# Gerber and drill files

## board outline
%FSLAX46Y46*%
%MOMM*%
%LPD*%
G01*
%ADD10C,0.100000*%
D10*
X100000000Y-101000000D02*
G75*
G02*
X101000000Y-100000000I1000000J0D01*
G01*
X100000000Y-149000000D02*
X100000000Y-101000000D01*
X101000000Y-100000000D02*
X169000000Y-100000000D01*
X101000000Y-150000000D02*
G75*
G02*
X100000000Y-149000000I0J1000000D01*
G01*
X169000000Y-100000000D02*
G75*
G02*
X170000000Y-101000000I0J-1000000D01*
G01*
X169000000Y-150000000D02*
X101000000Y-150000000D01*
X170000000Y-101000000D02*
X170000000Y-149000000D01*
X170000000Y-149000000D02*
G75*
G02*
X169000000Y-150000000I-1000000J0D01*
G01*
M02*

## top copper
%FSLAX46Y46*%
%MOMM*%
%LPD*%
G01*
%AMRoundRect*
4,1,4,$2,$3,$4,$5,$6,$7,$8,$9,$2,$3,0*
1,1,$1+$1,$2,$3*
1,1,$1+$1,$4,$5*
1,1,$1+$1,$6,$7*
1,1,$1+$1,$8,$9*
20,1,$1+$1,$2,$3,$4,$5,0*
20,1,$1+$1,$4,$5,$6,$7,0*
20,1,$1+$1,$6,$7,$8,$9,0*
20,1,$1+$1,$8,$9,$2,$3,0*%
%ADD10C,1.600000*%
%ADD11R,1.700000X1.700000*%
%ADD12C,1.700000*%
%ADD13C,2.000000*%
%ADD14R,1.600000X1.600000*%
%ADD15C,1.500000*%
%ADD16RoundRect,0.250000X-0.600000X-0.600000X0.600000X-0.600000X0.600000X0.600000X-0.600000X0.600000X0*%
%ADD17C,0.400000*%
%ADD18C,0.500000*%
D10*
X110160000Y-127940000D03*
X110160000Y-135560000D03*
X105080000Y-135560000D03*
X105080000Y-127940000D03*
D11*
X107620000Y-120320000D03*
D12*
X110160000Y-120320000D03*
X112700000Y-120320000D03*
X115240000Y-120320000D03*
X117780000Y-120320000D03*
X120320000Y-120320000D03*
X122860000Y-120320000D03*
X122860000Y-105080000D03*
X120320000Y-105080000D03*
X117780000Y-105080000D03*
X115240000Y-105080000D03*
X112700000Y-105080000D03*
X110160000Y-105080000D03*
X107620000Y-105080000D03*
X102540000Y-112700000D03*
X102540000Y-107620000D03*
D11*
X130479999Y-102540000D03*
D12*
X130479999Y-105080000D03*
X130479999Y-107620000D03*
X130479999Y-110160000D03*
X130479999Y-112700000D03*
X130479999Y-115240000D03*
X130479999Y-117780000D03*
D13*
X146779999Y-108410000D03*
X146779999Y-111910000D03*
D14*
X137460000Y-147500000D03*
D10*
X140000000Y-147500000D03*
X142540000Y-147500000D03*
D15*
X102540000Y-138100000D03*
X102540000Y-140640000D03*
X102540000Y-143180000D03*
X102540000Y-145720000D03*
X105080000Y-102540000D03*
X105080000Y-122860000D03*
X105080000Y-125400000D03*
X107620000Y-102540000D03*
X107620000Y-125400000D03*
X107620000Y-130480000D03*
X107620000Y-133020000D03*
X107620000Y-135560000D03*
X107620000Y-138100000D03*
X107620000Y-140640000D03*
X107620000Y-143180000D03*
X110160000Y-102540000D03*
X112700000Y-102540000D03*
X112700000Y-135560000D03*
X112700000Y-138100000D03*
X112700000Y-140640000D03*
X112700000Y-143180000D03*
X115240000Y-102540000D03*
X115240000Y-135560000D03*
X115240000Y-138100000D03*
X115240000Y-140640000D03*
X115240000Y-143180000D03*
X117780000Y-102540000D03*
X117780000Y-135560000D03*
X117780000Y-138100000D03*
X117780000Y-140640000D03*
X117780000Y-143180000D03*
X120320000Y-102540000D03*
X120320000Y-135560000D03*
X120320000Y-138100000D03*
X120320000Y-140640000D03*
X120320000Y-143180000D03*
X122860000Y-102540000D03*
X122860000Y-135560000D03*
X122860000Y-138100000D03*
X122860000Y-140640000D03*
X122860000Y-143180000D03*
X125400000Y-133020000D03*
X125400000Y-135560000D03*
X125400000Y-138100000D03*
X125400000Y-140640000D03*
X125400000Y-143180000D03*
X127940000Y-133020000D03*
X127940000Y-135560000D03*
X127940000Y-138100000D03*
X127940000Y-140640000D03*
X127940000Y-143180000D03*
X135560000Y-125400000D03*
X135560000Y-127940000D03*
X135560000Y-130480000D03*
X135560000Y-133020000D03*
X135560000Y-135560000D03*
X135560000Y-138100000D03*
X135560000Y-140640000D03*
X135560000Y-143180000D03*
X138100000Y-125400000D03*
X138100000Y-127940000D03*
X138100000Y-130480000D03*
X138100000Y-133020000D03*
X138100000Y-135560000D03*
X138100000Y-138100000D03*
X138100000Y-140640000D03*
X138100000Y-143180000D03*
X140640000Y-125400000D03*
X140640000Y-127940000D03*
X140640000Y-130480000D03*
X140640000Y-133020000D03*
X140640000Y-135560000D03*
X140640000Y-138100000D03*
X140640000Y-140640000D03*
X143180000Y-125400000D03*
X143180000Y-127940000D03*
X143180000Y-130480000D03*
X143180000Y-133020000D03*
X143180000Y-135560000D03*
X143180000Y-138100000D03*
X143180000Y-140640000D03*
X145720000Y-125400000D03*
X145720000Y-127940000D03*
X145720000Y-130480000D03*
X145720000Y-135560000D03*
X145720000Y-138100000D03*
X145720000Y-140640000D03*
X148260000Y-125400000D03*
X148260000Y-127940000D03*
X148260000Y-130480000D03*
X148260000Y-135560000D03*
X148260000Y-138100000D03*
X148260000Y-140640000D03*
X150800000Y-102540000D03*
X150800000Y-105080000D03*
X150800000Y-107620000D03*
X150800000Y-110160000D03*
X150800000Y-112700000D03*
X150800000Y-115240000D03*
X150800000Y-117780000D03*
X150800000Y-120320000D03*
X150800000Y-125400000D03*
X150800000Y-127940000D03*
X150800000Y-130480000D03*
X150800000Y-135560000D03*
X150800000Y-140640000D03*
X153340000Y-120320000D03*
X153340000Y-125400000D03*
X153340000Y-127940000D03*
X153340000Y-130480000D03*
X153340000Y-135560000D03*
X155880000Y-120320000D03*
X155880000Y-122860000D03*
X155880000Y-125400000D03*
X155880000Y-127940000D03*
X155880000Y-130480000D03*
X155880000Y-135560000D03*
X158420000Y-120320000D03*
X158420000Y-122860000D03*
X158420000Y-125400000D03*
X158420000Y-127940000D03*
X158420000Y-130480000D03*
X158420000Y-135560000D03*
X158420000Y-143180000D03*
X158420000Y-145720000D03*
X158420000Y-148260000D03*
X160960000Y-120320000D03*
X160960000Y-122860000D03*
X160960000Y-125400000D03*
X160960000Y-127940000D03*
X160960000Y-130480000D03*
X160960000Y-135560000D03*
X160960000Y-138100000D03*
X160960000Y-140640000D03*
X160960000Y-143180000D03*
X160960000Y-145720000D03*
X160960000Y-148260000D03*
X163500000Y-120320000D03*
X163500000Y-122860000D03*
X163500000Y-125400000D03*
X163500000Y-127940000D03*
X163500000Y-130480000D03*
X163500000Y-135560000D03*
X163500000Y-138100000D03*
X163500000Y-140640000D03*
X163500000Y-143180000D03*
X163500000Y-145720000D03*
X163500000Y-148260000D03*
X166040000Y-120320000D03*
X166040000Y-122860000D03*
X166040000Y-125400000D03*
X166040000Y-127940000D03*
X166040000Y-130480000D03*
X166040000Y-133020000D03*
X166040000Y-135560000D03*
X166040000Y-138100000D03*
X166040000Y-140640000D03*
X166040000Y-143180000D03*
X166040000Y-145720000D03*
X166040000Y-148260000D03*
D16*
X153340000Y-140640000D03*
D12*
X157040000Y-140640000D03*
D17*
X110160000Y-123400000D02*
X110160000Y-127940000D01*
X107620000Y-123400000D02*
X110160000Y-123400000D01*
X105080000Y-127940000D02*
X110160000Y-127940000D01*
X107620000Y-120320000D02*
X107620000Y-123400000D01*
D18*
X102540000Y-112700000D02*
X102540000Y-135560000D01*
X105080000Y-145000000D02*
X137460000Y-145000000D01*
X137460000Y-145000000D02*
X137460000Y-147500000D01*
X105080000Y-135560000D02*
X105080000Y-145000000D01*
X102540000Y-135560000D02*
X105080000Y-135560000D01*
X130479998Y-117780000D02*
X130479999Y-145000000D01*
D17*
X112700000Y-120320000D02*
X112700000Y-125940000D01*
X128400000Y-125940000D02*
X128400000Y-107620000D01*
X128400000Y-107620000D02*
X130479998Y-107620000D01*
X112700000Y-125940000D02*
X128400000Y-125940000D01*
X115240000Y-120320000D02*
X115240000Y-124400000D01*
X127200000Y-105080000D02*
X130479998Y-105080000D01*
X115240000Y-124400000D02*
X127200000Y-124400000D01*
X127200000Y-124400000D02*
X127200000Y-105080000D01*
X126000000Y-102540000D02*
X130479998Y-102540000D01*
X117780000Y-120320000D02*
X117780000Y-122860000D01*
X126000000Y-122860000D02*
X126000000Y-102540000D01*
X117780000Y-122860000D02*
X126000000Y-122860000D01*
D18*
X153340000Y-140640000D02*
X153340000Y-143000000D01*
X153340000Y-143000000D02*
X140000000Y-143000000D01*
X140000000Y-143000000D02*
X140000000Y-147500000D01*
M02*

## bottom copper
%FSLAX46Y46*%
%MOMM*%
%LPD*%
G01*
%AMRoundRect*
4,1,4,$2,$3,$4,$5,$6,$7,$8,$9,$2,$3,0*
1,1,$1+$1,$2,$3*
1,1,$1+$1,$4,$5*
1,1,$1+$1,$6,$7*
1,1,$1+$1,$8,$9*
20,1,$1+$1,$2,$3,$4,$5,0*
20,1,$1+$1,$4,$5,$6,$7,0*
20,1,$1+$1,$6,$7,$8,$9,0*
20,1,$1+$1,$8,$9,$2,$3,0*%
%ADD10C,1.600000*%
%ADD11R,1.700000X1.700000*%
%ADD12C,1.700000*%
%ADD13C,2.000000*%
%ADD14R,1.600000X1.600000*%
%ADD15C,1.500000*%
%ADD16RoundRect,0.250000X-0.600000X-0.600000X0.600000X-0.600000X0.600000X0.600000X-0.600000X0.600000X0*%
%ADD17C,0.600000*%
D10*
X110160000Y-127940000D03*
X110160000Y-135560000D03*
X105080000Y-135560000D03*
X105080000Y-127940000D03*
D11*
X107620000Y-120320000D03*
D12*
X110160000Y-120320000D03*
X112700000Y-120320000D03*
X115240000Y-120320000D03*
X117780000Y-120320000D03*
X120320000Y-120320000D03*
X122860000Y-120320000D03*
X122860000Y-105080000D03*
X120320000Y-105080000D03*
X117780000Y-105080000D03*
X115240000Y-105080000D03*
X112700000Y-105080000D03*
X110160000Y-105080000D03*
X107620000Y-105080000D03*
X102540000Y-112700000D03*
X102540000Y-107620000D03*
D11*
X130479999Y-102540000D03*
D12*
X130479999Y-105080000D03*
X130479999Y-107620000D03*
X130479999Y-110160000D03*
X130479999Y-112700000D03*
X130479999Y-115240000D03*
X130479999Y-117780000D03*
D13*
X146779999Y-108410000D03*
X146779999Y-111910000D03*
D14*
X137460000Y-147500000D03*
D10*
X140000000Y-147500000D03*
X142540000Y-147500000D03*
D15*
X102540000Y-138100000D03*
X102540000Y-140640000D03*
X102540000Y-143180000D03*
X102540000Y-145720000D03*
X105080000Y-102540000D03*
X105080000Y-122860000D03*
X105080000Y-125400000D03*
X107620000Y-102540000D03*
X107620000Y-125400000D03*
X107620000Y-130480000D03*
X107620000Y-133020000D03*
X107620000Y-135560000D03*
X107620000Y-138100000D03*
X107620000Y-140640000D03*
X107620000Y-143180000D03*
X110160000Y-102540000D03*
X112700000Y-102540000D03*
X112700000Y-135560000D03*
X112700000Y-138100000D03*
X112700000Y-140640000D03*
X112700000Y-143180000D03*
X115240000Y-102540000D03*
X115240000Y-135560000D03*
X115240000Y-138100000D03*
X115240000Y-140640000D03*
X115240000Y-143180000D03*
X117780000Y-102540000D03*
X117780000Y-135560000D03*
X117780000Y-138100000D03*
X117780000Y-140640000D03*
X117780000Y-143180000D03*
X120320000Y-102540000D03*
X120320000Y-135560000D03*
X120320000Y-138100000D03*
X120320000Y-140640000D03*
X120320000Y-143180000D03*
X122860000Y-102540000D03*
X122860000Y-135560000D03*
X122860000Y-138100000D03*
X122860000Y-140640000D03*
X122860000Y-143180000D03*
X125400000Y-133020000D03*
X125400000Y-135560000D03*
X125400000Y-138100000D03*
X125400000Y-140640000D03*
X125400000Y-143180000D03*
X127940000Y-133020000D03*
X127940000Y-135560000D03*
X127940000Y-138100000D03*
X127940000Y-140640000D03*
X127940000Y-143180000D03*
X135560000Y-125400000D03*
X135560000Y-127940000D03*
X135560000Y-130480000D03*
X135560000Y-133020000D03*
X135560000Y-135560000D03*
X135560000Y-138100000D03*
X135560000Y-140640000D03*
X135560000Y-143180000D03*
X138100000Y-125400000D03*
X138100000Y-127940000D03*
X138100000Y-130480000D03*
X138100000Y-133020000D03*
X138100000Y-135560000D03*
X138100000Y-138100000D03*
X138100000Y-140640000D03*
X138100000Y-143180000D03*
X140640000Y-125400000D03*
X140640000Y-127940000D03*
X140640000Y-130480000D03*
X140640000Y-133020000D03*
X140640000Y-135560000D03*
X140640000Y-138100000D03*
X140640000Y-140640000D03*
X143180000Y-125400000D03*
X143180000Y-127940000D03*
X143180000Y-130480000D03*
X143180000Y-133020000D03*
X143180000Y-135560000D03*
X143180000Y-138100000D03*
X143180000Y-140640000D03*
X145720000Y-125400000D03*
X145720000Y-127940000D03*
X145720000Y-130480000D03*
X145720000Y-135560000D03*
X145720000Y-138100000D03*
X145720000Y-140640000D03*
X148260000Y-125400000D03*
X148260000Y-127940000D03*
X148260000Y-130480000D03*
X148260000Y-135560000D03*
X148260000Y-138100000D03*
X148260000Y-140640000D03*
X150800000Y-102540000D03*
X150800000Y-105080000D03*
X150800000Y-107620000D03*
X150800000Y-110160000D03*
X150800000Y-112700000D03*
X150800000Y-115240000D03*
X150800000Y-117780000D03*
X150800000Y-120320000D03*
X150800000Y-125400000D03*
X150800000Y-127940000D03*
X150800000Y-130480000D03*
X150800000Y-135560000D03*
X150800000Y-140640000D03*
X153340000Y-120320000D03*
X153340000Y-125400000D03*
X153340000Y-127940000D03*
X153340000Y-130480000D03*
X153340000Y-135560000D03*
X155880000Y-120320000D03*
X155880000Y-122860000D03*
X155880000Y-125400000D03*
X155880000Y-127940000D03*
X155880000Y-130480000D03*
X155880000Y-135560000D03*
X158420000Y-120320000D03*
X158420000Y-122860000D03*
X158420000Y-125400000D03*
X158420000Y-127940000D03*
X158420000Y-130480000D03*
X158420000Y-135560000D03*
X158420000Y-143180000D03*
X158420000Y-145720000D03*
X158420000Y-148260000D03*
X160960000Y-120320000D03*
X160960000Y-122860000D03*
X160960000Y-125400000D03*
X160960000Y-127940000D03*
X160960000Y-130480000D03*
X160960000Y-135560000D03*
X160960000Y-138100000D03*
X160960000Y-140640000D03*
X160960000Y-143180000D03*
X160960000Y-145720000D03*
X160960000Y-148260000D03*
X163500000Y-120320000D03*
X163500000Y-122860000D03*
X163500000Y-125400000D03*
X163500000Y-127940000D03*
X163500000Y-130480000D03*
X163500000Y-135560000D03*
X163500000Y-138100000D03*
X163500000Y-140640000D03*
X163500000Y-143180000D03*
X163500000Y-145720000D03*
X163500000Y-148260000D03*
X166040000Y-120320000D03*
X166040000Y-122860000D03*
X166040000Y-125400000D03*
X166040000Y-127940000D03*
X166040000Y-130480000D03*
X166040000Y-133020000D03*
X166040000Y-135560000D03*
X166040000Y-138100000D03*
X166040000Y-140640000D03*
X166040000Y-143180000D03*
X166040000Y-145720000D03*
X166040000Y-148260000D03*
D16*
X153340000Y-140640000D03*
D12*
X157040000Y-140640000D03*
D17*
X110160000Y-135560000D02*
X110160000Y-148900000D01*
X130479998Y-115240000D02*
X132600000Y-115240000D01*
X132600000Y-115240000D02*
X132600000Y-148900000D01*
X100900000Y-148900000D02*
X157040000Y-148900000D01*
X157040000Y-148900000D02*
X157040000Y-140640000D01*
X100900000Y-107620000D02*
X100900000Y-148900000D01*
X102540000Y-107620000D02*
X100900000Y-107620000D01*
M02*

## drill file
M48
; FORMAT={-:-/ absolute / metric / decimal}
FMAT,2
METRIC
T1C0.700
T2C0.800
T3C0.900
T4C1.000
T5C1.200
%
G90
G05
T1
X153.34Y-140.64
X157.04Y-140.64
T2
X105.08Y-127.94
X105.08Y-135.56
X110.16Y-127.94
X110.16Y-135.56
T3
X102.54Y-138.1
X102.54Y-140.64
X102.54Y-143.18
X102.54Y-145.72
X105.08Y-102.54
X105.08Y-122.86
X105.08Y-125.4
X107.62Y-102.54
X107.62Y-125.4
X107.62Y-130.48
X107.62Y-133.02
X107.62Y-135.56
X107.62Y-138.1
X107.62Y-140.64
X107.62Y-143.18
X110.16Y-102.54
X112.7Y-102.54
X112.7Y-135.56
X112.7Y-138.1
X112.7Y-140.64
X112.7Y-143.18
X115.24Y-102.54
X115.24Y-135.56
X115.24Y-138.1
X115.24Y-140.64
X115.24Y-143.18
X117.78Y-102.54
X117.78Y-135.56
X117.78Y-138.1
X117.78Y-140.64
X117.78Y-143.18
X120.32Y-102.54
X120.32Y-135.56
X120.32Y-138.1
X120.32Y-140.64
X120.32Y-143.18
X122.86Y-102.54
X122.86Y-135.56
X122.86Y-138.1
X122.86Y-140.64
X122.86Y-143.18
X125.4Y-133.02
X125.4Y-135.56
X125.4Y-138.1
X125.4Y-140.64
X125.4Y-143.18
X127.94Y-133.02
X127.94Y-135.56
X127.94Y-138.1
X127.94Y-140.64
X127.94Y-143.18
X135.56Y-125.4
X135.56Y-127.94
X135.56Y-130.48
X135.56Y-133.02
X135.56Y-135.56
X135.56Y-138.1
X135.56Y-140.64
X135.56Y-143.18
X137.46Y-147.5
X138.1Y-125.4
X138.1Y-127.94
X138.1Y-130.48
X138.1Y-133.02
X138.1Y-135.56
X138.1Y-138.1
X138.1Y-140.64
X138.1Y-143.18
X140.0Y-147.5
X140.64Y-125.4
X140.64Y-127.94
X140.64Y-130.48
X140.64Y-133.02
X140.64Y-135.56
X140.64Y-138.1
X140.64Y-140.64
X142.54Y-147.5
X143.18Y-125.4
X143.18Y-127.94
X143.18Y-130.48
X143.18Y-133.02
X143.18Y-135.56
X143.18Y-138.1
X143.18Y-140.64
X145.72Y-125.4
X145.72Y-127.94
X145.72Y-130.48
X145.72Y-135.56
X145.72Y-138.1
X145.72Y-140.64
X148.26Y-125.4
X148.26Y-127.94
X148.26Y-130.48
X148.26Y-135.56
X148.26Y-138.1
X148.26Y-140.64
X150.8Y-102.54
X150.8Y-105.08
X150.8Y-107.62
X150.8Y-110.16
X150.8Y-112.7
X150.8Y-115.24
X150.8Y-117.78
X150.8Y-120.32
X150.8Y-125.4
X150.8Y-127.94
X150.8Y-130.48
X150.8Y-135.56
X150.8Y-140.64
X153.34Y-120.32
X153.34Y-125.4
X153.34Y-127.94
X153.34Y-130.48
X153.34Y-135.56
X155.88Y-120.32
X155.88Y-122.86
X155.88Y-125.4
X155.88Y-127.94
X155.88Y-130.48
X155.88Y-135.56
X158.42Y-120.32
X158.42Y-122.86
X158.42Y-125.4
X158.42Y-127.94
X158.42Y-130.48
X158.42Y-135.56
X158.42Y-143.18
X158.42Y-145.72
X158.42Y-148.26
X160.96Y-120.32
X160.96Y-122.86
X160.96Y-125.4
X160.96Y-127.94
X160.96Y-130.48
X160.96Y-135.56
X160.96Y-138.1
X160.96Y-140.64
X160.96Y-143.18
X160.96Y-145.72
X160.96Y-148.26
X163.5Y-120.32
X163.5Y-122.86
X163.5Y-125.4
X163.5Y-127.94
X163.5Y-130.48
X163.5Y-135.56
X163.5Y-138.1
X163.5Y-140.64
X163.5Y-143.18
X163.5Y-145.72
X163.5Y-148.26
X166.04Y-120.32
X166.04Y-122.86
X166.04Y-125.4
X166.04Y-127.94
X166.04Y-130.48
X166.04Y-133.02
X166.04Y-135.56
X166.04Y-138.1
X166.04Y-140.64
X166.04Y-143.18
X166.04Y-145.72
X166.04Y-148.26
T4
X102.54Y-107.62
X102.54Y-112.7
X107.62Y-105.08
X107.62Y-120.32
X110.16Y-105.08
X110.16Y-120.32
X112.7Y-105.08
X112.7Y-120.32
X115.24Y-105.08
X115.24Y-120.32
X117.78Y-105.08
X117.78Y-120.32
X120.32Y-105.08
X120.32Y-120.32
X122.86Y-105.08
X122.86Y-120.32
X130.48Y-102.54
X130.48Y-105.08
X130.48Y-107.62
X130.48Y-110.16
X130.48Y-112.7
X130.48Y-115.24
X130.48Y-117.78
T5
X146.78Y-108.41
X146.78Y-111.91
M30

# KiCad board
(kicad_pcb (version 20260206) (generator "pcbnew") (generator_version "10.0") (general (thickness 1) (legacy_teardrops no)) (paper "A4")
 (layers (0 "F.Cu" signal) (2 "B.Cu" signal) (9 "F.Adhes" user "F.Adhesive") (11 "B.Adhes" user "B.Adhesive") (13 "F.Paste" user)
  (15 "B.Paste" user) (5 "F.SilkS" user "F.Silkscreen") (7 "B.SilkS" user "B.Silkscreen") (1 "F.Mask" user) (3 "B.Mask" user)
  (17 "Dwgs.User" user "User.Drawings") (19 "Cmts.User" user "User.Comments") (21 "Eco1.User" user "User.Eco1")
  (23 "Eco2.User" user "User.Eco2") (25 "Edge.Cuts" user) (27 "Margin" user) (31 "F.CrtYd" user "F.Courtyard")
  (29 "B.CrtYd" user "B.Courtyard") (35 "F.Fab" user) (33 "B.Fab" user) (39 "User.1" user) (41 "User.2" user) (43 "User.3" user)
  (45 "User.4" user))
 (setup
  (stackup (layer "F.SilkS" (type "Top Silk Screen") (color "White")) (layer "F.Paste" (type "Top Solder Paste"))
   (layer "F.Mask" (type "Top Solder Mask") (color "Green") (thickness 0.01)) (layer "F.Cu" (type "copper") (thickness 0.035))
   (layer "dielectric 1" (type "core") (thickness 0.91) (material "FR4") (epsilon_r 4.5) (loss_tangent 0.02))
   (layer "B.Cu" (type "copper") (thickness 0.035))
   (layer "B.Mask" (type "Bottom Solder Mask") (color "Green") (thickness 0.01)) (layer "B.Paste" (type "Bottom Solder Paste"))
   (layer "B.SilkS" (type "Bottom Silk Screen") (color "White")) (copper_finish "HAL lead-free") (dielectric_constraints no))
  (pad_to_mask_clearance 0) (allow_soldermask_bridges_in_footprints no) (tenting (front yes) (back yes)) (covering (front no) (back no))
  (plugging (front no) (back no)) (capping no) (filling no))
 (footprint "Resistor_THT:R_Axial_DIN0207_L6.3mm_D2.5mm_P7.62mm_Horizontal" (layer "F.Cu") (at 110.16 127.94 -90)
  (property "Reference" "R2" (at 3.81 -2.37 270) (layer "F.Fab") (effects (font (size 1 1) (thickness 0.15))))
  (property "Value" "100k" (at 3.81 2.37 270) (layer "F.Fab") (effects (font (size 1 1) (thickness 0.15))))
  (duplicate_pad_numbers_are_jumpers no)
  (pad "1" thru_hole circle (at 0 0 270) (size 1.6 1.6) (drill 0.8) (layers "*.Cu" "*.Mask") (remove_unused_layers no) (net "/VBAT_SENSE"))
  (pad "2" thru_hole circle (at 7.62 0 270) (size 1.6 1.6) (drill 0.8) (layers "*.Cu" "*.Mask") (remove_unused_layers no) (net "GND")))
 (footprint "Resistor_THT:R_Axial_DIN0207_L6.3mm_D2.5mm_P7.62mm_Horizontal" (layer "F.Cu") (at 105.08 135.56 90)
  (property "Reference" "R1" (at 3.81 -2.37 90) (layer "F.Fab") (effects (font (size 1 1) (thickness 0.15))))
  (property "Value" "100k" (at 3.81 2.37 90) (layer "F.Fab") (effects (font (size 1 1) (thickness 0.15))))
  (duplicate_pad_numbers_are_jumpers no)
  (pad "1" thru_hole circle (at 0 0 90) (size 1.6 1.6) (drill 0.8) (layers "*.Cu" "*.Mask") (remove_unused_layers no) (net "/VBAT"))
  (pad "2" thru_hole circle (at 7.62 0 90) (size 1.6 1.6) (drill 0.8) (layers "*.Cu" "*.Mask") (remove_unused_layers no) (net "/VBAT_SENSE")))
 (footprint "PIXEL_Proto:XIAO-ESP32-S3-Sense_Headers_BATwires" (layer "F.Cu") (at 115.24 112.7 180)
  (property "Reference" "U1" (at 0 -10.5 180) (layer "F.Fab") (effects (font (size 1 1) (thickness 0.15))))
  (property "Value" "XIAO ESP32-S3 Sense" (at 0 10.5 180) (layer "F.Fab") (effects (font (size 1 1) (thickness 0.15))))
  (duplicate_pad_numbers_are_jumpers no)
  (pad "1" thru_hole rect (at 7.62 -7.62 180) (size 1.7 1.7) (drill 1) (layers "*.Cu" "*.Mask") (remove_unused_layers no)
   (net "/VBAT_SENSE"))
  (pad "2" thru_hole circle (at 5.08 -7.62 180) (size 1.7 1.7) (drill 1) (layers "*.Cu" "*.Mask") (remove_unused_layers no)
   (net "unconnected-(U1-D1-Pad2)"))
  (pad "3" thru_hole circle (at 2.54 -7.62 180) (size 1.7 1.7) (drill 1) (layers "*.Cu" "*.Mask") (remove_unused_layers no)
   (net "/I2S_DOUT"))
  (pad "4" thru_hole circle (at 0 -7.62 180) (size 1.7 1.7) (drill 1) (layers "*.Cu" "*.Mask") (remove_unused_layers no) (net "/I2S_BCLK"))
  (pad "5" thru_hole circle (at -2.54 -7.62 180) (size 1.7 1.7) (drill 1) (layers "*.Cu" "*.Mask") (remove_unused_layers no)
   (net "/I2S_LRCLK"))
  (pad "6" thru_hole circle (at -5.08 -7.62 180) (size 1.7 1.7) (drill 1) (layers "*.Cu" "*.Mask") (remove_unused_layers no)
   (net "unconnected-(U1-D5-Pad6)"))
  (pad "7" thru_hole circle (at -7.62 -7.62 180) (size 1.7 1.7) (drill 1) (layers "*.Cu" "*.Mask") (remove_unused_layers no)
   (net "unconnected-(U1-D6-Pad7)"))
  (pad "8" thru_hole circle (at -7.62 7.62 180) (size 1.7 1.7) (drill 1) (layers "*.Cu" "*.Mask") (remove_unused_layers no)
   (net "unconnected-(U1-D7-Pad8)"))
  (pad "9" thru_hole circle (at -5.08 7.62 180) (size 1.7 1.7) (drill 1) (layers "*.Cu" "*.Mask") (remove_unused_layers no)
   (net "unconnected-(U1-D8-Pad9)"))
  (pad "10" thru_hole circle (at -2.54 7.62 180) (size 1.7 1.7) (drill 1) (layers "*.Cu" "*.Mask") (remove_unused_layers no)
   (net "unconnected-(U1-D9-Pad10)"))
  (pad "11" thru_hole circle (at 0 7.62 180) (size 1.7 1.7) (drill 1) (layers "*.Cu" "*.Mask") (remove_unused_layers no)
   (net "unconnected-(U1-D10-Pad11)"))
  (pad "12" thru_hole circle (at 2.54 7.62 180) (size 1.7 1.7) (drill 1) (layers "*.Cu" "*.Mask") (remove_unused_layers no)
   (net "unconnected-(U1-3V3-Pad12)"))
  (pad "13" thru_hole circle (at 5.08 7.62 180) (size 1.7 1.7) (drill 1) (layers "*.Cu" "*.Mask") (remove_unused_layers no)
   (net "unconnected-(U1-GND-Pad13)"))
  (pad "14" thru_hole circle (at 7.62 7.62 180) (size 1.7 1.7) (drill 1) (layers "*.Cu" "*.Mask") (remove_unused_layers no)
   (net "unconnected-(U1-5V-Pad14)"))
  (pad "23" thru_hole circle (at 12.7 0 180) (size 1.7 1.7) (drill 1) (layers "*.Cu" "*.Mask") (remove_unused_layers no) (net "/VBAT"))
  (pad "24" thru_hole circle (at 12.7 5.08 180) (size 1.7 1.7) (drill 1) (layers "*.Cu" "*.Mask") (remove_unused_layers no) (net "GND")))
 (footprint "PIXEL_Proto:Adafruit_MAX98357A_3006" (layer "F.Cu") (at 130.479999 102.54)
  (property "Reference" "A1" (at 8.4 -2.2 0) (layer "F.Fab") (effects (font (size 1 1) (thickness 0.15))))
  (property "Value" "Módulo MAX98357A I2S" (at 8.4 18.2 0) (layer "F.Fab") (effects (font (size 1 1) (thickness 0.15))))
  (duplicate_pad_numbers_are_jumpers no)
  (pad "1" thru_hole rect (at 0 0) (size 1.7 1.7) (drill 1) (layers "*.Cu" "*.Mask") (remove_unused_layers no) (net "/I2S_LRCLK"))
  (pad "2" thru_hole circle (at 0 2.54) (size 1.7 1.7) (drill 1) (layers "*.Cu" "*.Mask") (remove_unused_layers no) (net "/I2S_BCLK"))
  (pad "3" thru_hole circle (at 0 5.08) (size 1.7 1.7) (drill 1) (layers "*.Cu" "*.Mask") (remove_unused_layers no) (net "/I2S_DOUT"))
  (pad "4" thru_hole circle (at 0 7.62) (size 1.7 1.7) (drill 1) (layers "*.Cu" "*.Mask") (remove_unused_layers no)
   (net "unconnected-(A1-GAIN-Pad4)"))
  (pad "5" thru_hole circle (at 0 10.16) (size 1.7 1.7) (drill 1) (layers "*.Cu" "*.Mask") (remove_unused_layers no)
   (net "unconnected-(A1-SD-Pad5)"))
  (pad "6" thru_hole circle (at 0 12.7) (size 1.7 1.7) (drill 1) (layers "*.Cu" "*.Mask") (remove_unused_layers no) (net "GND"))
  (pad "7" thru_hole circle (at 0 15.24) (size 1.7 1.7) (drill 1) (layers "*.Cu" "*.Mask") (remove_unused_layers no) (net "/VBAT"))
  (pad "8" thru_hole circle (at 16.3 5.87) (size 2 2) (drill 1.2) (layers "*.Cu" "*.Mask") (remove_unused_layers no) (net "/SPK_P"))
  (pad "9" thru_hole circle (at 16.3 9.37) (size 2 2) (drill 1.2) (layers "*.Cu" "*.Mask") (remove_unused_layers no) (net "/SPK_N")))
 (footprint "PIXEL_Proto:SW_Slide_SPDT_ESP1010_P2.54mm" (layer "F.Cu") (at 140 147.5)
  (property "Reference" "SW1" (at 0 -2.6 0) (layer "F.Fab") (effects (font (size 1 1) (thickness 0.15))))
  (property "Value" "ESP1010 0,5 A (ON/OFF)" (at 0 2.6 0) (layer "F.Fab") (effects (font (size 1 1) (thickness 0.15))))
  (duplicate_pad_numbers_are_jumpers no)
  (pad "1" thru_hole rect (at -2.54 0) (size 1.6 1.6) (drill 0.9) (layers "*.Cu" "*.Mask") (remove_unused_layers no) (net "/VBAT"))
  (pad "2" thru_hole circle (at 0 0) (size 1.6 1.6) (drill 0.9) (layers "*.Cu" "*.Mask") (remove_unused_layers no) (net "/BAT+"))
  (pad "3" thru_hole circle (at 2.54 0) (size 1.6 1.6) (drill 0.9) (layers "*.Cu" "*.Mask") (remove_unused_layers no)
   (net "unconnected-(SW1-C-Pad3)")))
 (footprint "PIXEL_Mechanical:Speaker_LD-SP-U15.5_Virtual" (layer "F.Cu") (at 161 108.2)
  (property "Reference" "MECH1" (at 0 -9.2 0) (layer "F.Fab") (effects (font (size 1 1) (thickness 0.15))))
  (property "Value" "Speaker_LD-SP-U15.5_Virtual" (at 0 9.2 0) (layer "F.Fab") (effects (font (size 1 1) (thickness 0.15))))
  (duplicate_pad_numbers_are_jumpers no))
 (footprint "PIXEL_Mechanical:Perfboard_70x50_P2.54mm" (layer "F.Cu") (at 0 0)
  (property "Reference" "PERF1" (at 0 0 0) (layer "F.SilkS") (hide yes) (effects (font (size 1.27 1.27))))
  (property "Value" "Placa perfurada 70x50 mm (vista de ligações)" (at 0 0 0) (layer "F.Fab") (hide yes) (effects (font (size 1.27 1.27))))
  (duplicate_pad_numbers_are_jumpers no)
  (pad "" thru_hole circle (at 102.54 138.1) (size 1.5 1.5) (drill 0.9) (layers "*.Cu" "*.Mask") (remove_unused_layers no))
  (pad "" thru_hole circle (at 102.54 140.64) (size 1.5 1.5) (drill 0.9) (layers "*.Cu" "*.Mask") (remove_unused_layers no))
  (pad "" thru_hole circle (at 102.54 143.18) (size 1.5 1.5) (drill 0.9) (layers "*.Cu" "*.Mask") (remove_unused_layers no))
  (pad "" thru_hole circle (at 102.54 145.72) (size 1.5 1.5) (drill 0.9) (layers "*.Cu" "*.Mask") (remove_unused_layers no))
  (pad "" thru_hole circle (at 105.08 102.54) (size 1.5 1.5) (drill 0.9) (layers "*.Cu" "*.Mask") (remove_unused_layers no))
  (pad "" thru_hole circle (at 105.08 122.86) (size 1.5 1.5) (drill 0.9) (layers "*.Cu" "*.Mask") (remove_unused_layers no))
  (pad "" thru_hole circle (at 105.08 125.4) (size 1.5 1.5) (drill 0.9) (layers "*.Cu" "*.Mask") (remove_unused_layers no))
  (pad "" thru_hole circle (at 107.62 102.54) (size 1.5 1.5) (drill 0.9) (layers "*.Cu" "*.Mask") (remove_unused_layers no))
  (pad "" thru_hole circle (at 107.62 125.4) (size 1.5 1.5) (drill 0.9) (layers "*.Cu" "*.Mask") (remove_unused_layers no))
  (pad "" thru_hole circle (at 107.62 130.48) (size 1.5 1.5) (drill 0.9) (layers "*.Cu" "*.Mask") (remove_unused_layers no))
  (pad "" thru_hole circle (at 107.62 133.02) (size 1.5 1.5) (drill 0.9) (layers "*.Cu" "*.Mask") (remove_unused_layers no))
  (pad "" thru_hole circle (at 107.62 135.56) (size 1.5 1.5) (drill 0.9) (layers "*.Cu" "*.Mask") (remove_unused_layers no))
  (pad "" thru_hole circle (at 107.62 138.1) (size 1.5 1.5) (drill 0.9) (layers "*.Cu" "*.Mask") (remove_unused_layers no))
  (pad "" thru_hole circle (at 107.62 140.64) (size 1.5 1.5) (drill 0.9) (layers "*.Cu" "*.Mask") (remove_unused_layers no))
  (pad "" thru_hole circle (at 107.62 143.18) (size 1.5 1.5) (drill 0.9) (layers "*.Cu" "*.Mask") (remove_unused_layers no))
  (pad "" thru_hole circle (at 110.16 102.54) (size 1.5 1.5) (drill 0.9) (layers "*.Cu" "*.Mask") (remove_unused_layers no))
  (pad "" thru_hole circle (at 112.7 102.54) (size 1.5 1.5) (drill 0.9) (layers "*.Cu" "*.Mask") (remove_unused_layers no))
  (pad "" thru_hole circle (at 112.7 135.56) (size 1.5 1.5) (drill 0.9) (layers "*.Cu" "*.Mask") (remove_unused_layers no))
  (pad "" thru_hole circle (at 112.7 138.1) (size 1.5 1.5) (drill 0.9) (layers "*.Cu" "*.Mask") (remove_unused_layers no))
  (pad "" thru_hole circle (at 112.7 140.64) (size 1.5 1.5) (drill 0.9) (layers "*.Cu" "*.Mask") (remove_unused_layers no))
  (pad "" thru_hole circle (at 112.7 143.18) (size 1.5 1.5) (drill 0.9) (layers "*.Cu" "*.Mask") (remove_unused_layers no))
  (pad "" thru_hole circle (at 115.24 102.54) (size 1.5 1.5) (drill 0.9) (layers "*.Cu" "*.Mask") (remove_unused_layers no))
  (pad "" thru_hole circle (at 115.24 135.56) (size 1.5 1.5) (drill 0.9) (layers "*.Cu" "*.Mask") (remove_unused_layers no))
  (pad "" thru_hole circle (at 115.24 138.1) (size 1.5 1.5) (drill 0.9) (layers "*.Cu" "*.Mask") (remove_unused_layers no))
  (pad "" thru_hole circle (at 115.24 140.64) (size 1.5 1.5) (drill 0.9) (layers "*.Cu" "*.Mask") (remove_unused_layers no))
  (pad "" thru_hole circle (at 115.24 143.18) (size 1.5 1.5) (drill 0.9) (layers "*.Cu" "*.Mask") (remove_unused_layers no))
  (pad "" thru_hole circle (at 117.78 102.54) (size 1.5 1.5) (drill 0.9) (layers "*.Cu" "*.Mask") (remove_unused_layers no))
  (pad "" thru_hole circle (at 117.78 135.56) (size 1.5 1.5) (drill 0.9) (layers "*.Cu" "*.Mask") (remove_unused_layers no))
  (pad "" thru_hole circle (at 117.78 138.1) (size 1.5 1.5) (drill 0.9) (layers "*.Cu" "*.Mask") (remove_unused_layers no))
  (pad "" thru_hole circle (at 117.78 140.64) (size 1.5 1.5) (drill 0.9) (layers "*.Cu" "*.Mask") (remove_unused_layers no))
  (pad "" thru_hole circle (at 117.78 143.18) (size 1.5 1.5) (drill 0.9) (layers "*.Cu" "*.Mask") (remove_unused_layers no))
  (pad "" thru_hole circle (at 120.32 102.54) (size 1.5 1.5) (drill 0.9) (layers "*.Cu" "*.Mask") (remove_unused_layers no))
  (pad "" thru_hole circle (at 120.32 135.56) (size 1.5 1.5) (drill 0.9) (layers "*.Cu" "*.Mask") (remove_unused_layers no))
  (pad "" thru_hole circle (at 120.32 138.1) (size 1.5 1.5) (drill 0.9) (layers "*.Cu" "*.Mask") (remove_unused_layers no))
  (pad "" thru_hole circle (at 120.32 140.64) (size 1.5 1.5) (drill 0.9) (layers "*.Cu" "*.Mask") (remove_unused_layers no))
  (pad "" thru_hole circle (at 120.32 143.18) (size 1.5 1.5) (drill 0.9) (layers "*.Cu" "*.Mask") (remove_unused_layers no))
  (pad "" thru_hole circle (at 122.86 102.54) (size 1.5 1.5) (drill 0.9) (layers "*.Cu" "*.Mask") (remove_unused_layers no))
  (pad "" thru_hole circle (at 122.86 135.56) (size 1.5 1.5) (drill 0.9) (layers "*.Cu" "*.Mask") (remove_unused_layers no))
  (pad "" thru_hole circle (at 122.86 138.1) (size 1.5 1.5) (drill 0.9) (layers "*.Cu" "*.Mask") (remove_unused_layers no))
  (pad "" thru_hole circle (at 122.86 140.64) (size 1.5 1.5) (drill 0.9) (layers "*.Cu" "*.Mask") (remove_unused_layers no))
  (pad "" thru_hole circle (at 122.86 143.18) (size 1.5 1.5) (drill 0.9) (layers "*.Cu" "*.Mask") (remove_unused_layers no))
  (pad "" thru_hole circle (at 125.4 133.02) (size 1.5 1.5) (drill 0.9) (layers "*.Cu" "*.Mask") (remove_unused_layers no))
  (pad "" thru_hole circle (at 125.4 135.56) (size 1.5 1.5) (drill 0.9) (layers "*.Cu" "*.Mask") (remove_unused_layers no))
  (pad "" thru_hole circle (at 125.4 138.1) (size 1.5 1.5) (drill 0.9) (layers "*.Cu" "*.Mask") (remove_unused_layers no))
  (pad "" thru_hole circle (at 125.4 140.64) (size 1.5 1.5) (drill 0.9) (layers "*.Cu" "*.Mask") (remove_unused_layers no))
  (pad "" thru_hole circle (at 125.4 143.18) (size 1.5 1.5) (drill 0.9) (layers "*.Cu" "*.Mask") (remove_unused_layers no))
  (pad "" thru_hole circle (at 127.94 133.02) (size 1.5 1.5) (drill 0.9) (layers "*.Cu" "*.Mask") (remove_unused_layers no))
  (pad "" thru_hole circle (at 127.94 135.56) (size 1.5 1.5) (drill 0.9) (layers "*.Cu" "*.Mask") (remove_unused_layers no))
  (pad "" thru_hole circle (at 127.94 138.1) (size 1.5 1.5) (drill 0.9) (layers "*.Cu" "*.Mask") (remove_unused_layers no))
  (pad "" thru_hole circle (at 127.94 140.64) (size 1.5 1.5) (drill 0.9) (layers "*.Cu" "*.Mask") (remove_unused_layers no))
  (pad "" thru_hole circle (at 127.94 143.18) (size 1.5 1.5) (drill 0.9) (layers "*.Cu" "*.Mask") (remove_unused_layers no))
  (pad "" thru_hole circle (at 135.56 125.4) (size 1.5 1.5) (drill 0.9) (layers "*.Cu" "*.Mask") (remove_unused_layers no))
  (pad "" thru_hole circle (at 135.56 127.94) (size 1.5 1.5) (drill 0.9) (layers "*.Cu" "*.Mask") (remove_unused_layers no))
  (pad "" thru_hole circle (at 135.56 130.48) (size 1.5 1.5) (drill 0.9) (layers "*.Cu" "*.Mask") (remove_unused_layers no))
  (pad "" thru_hole circle (at 135.56 133.02) (size 1.5 1.5) (drill 0.9) (layers "*.Cu" "*.Mask") (remove_unused_layers no))
  (pad "" thru_hole circle (at 135.56 135.56) (size 1.5 1.5) (drill 0.9) (layers "*.Cu" "*.Mask") (remove_unused_layers no))
  (pad "" thru_hole circle (at 135.56 138.1) (size 1.5 1.5) (drill 0.9) (layers "*.Cu" "*.Mask") (remove_unused_layers no))
  (pad "" thru_hole circle (at 135.56 140.64) (size 1.5 1.5) (drill 0.9) (layers "*.Cu" "*.Mask") (remove_unused_layers no))
  (pad "" thru_hole circle (at 135.56 143.18) (size 1.5 1.5) (drill 0.9) (layers "*.Cu" "*.Mask") (remove_unused_layers no))
  (pad "" thru_hole circle (at 138.1 125.4) (size 1.5 1.5) (drill 0.9) (layers "*.Cu" "*.Mask") (remove_unused_layers no))
  (pad "" thru_hole circle (at 138.1 127.94) (size 1.5 1.5) (drill 0.9) (layers "*.Cu" "*.Mask") (remove_unused_layers no))
  (pad "" thru_hole circle (at 138.1 130.48) (size 1.5 1.5) (drill 0.9) (layers "*.Cu" "*.Mask") (remove_unused_layers no))
  (pad "" thru_hole circle (at 138.1 133.02) (size 1.5 1.5) (drill 0.9) (layers "*.Cu" "*.Mask") (remove_unused_layers no))
  (pad "" thru_hole circle (at 138.1 135.56) (size 1.5 1.5) (drill 0.9) (layers "*.Cu" "*.Mask") (remove_unused_layers no))
  (pad "" thru_hole circle (at 138.1 138.1) (size 1.5 1.5) (drill 0.9) (layers "*.Cu" "*.Mask") (remove_unused_layers no))
  (pad "" thru_hole circle (at 138.1 140.64) (size 1.5 1.5) (drill 0.9) (layers "*.Cu" "*.Mask") (remove_unused_layers no))
  (pad "" thru_hole circle (at 138.1 143.18) (size 1.5 1.5) (drill 0.9) (layers "*.Cu" "*.Mask") (remove_unused_layers no))
  (pad "" thru_hole circle (at 140.64 125.4) (size 1.5 1.5) (drill 0.9) (layers "*.Cu" "*.Mask") (remove_unused_layers no))
  (pad "" thru_hole circle (at 140.64 127.94) (size 1.5 1.5) (drill 0.9) (layers "*.Cu" "*.Mask") (remove_unused_layers no))
  (pad "" thru_hole circle (at 140.64 130.48) (size 1.5 1.5) (drill 0.9) (layers "*.Cu" "*.Mask") (remove_unused_layers no))
  (pad "" thru_hole circle (at 140.64 133.02) (size 1.5 1.5) (drill 0.9) (layers "*.Cu" "*.Mask") (remove_unused_layers no))
  (pad "" thru_hole circle (at 140.64 135.56) (size 1.5 1.5) (drill 0.9) (layers "*.Cu" "*.Mask") (remove_unused_layers no))
  (pad "" thru_hole circle (at 140.64 138.1) (size 1.5 1.5) (drill 0.9) (layers "*.Cu" "*.Mask") (remove_unused_layers no))
  (pad "" thru_hole circle (at 140.64 140.64) (size 1.5 1.5) (drill 0.9) (layers "*.Cu" "*.Mask") (remove_unused_layers no))
  (pad "" thru_hole circle (at 143.18 125.4) (size 1.5 1.5) (drill 0.9) (layers "*.Cu" "*.Mask") (remove_unused_layers no))
  (pad "" thru_hole circle (at 143.18 127.94) (size 1.5 1.5) (drill 0.9) (layers "*.Cu" "*.Mask") (remove_unused_layers no))
  (pad "" thru_hole circle (at 143.18 130.48) (size 1.5 1.5) (drill 0.9) (layers "*.Cu" "*.Mask") (remove_unused_layers no))
  (pad "" thru_hole circle (at 143.18 133.02) (size 1.5 1.5) (drill 0.9) (layers "*.Cu" "*.Mask") (remove_unused_layers no))
  (pad "" thru_hole circle (at 143.18 135.56) (size 1.5 1.5) (drill 0.9) (layers "*.Cu" "*.Mask") (remove_unused_layers no))
  (pad "" thru_hole circle (at 143.18 138.1) (size 1.5 1.5) (drill 0.9) (layers "*.Cu" "*.Mask") (remove_unused_layers no))
  (pad "" thru_hole circle (at 143.18 140.64) (size 1.5 1.5) (drill 0.9) (layers "*.Cu" "*.Mask") (remove_unused_layers no))
  (pad "" thru_hole circle (at 145.72 125.4) (size 1.5 1.5) (drill 0.9) (layers "*.Cu" "*.Mask") (remove_unused_layers no))
  (pad "" thru_hole circle (at 145.72 127.94) (size 1.5 1.5) (drill 0.9) (layers "*.Cu" "*.Mask") (remove_unused_layers no))
  (pad "" thru_hole circle (at 145.72 130.48) (size 1.5 1.5) (drill 0.9) (layers "*.Cu" "*.Mask") (remove_unused_layers no))
  (pad "" thru_hole circle (at 145.72 135.56) (size 1.5 1.5) (drill 0.9) (layers "*.Cu" "*.Mask") (remove_unused_layers no))
  (pad "" thru_hole circle (at 145.72 138.1) (size 1.5 1.5) (drill 0.9) (layers "*.Cu" "*.Mask") (remove_unused_layers no))
  (pad "" thru_hole circle (at 145.72 140.64) (size 1.5 1.5) (drill 0.9) (layers "*.Cu" "*.Mask") (remove_unused_layers no))
  (pad "" thru_hole circle (at 148.26 125.4) (size 1.5 1.5) (drill 0.9) (layers "*.Cu" "*.Mask") (remove_unused_layers no))
  (pad "" thru_hole circle (at 148.26 127.94) (size 1.5 1.5) (drill 0.9) (layers "*.Cu" "*.Mask") (remove_unused_layers no))
  (pad "" thru_hole circle (at 148.26 130.48) (size 1.5 1.5) (drill 0.9) (layers "*.Cu" "*.Mask") (remove_unused_layers no))
  (pad "" thru_hole circle (at 148.26 135.56) (size 1.5 1.5) (drill 0.9) (layers "*.Cu" "*.Mask") (remove_unused_layers no))
  (pad "" thru_hole circle (at 148.26 138.1) (size 1.5 1.5) (drill 0.9) (layers "*.Cu" "*.Mask") (remove_unused_layers no))
  (pad "" thru_hole circle (at 148.26 140.64) (size 1.5 1.5) (drill 0.9) (layers "*.Cu" "*.Mask") (remove_unused_layers no))
  (pad "" thru_hole circle (at 150.8 102.54) (size 1.5 1.5) (drill 0.9) (layers "*.Cu" "*.Mask") (remove_unused_layers no))
  (pad "" thru_hole circle (at 150.8 105.08) (size 1.5 1.5) (drill 0.9) (layers "*.Cu" "*.Mask") (remove_unused_layers no))
  (pad "" thru_hole circle (at 150.8 107.62) (size 1.5 1.5) (drill 0.9) (layers "*.Cu" "*.Mask") (remove_unused_layers no))
  (pad "" thru_hole circle (at 150.8 110.16) (size 1.5 1.5) (drill 0.9) (layers "*.Cu" "*.Mask") (remove_unused_layers no))
  (pad "" thru_hole circle (at 150.8 112.7) (size 1.5 1.5) (drill 0.9) (layers "*.Cu" "*.Mask") (remove_unused_layers no))
  (pad "" thru_hole circle (at 150.8 115.24) (size 1.5 1.5) (drill 0.9) (layers "*.Cu" "*.Mask") (remove_unused_layers no))
  (pad "" thru_hole circle (at 150.8 117.78) (size 1.5 1.5) (drill 0.9) (layers "*.Cu" "*.Mask") (remove_unused_layers no))
  (pad "" thru_hole circle (at 150.8 120.32) (size 1.5 1.5) (drill 0.9) (layers "*.Cu" "*.Mask") (remove_unused_layers no))
  (pad "" thru_hole circle (at 150.8 125.4) (size 1.5 1.5) (drill 0.9) (layers "*.Cu" "*.Mask") (remove_unused_layers no))
  (pad "" thru_hole circle (at 150.8 127.94) (size 1.5 1.5) (drill 0.9) (layers "*.Cu" "*.Mask") (remove_unused_layers no))
  (pad "" thru_hole circle (at 150.8 130.48) (size 1.5 1.5) (drill 0.9) (layers "*.Cu" "*.Mask") (remove_unused_layers no))
  (pad "" thru_hole circle (at 150.8 135.56) (size 1.5 1.5) (drill 0.9) (layers "*.Cu" "*.Mask") (remove_unused_layers no))
  (pad "" thru_hole circle (at 150.8 140.64) (size 1.5 1.5) (drill 0.9) (layers "*.Cu" "*.Mask") (remove_unused_layers no))
  (pad "" thru_hole circle (at 153.34 120.32) (size 1.5 1.5) (drill 0.9) (layers "*.Cu" "*.Mask") (remove_unused_layers no))
  (pad "" thru_hole circle (at 153.34 125.4) (size 1.5 1.5) (drill 0.9) (layers "*.Cu" "*.Mask") (remove_unused_layers no))
  (pad "" thru_hole circle (at 153.34 127.94) (size 1.5 1.5) (drill 0.9) (layers "*.Cu" "*.Mask") (remove_unused_layers no))
  (pad "" thru_hole circle (at 153.34 130.48) (size 1.5 1.5) (drill 0.9) (layers "*.Cu" "*.Mask") (remove_unused_layers no))
  (pad "" thru_hole circle (at 153.34 135.56) (size 1.5 1.5) (drill 0.9) (layers "*.Cu" "*.Mask") (remove_unused_layers no))
  (pad "" thru_hole circle (at 155.88 120.32) (size 1.5 1.5) (drill 0.9) (layers "*.Cu" "*.Mask") (remove_unused_layers no))
  (pad "" thru_hole circle (at 155.88 122.86) (size 1.5 1.5) (drill 0.9) (layers "*.Cu" "*.Mask") (remove_unused_layers no))
  (pad "" thru_hole circle (at 155.88 125.4) (size 1.5 1.5) (drill 0.9) (layers "*.Cu" "*.Mask") (remove_unused_layers no))
  (pad "" thru_hole circle (at 155.88 127.94) (size 1.5 1.5) (drill 0.9) (layers "*.Cu" "*.Mask") (remove_unused_layers no))
  (pad "" thru_hole circle (at 155.88 130.48) (size 1.5 1.5) (drill 0.9) (layers "*.Cu" "*.Mask") (remove_unused_layers no))
  (pad "" thru_hole circle (at 155.88 135.56) (size 1.5 1.5) (drill 0.9) (layers "*.Cu" "*.Mask") (remove_unused_layers no))
  (pad "" thru_hole circle (at 158.42 120.32) (size 1.5 1.5) (drill 0.9) (layers "*.Cu" "*.Mask") (remove_unused_layers no))
  (pad "" thru_hole circle (at 158.42 122.86) (size 1.5 1.5) (drill 0.9) (layers "*.Cu" "*.Mask") (remove_unused_layers no))
  (pad "" thru_hole circle (at 158.42 125.4) (size 1.5 1.5) (drill 0.9) (layers "*.Cu" "*.Mask") (remove_unused_layers no))
  (pad "" thru_hole circle (at 158.42 127.94) (size 1.5 1.5) (drill 0.9) (layers "*.Cu" "*.Mask") (remove_unused_layers no))
  (pad "" thru_hole circle (at 158.42 130.48) (size 1.5 1.5) (drill 0.9) (layers "*.Cu" "*.Mask") (remove_unused_layers no))
  (pad "" thru_hole circle (at 158.42 135.56) (size 1.5 1.5) (drill 0.9) (layers "*.Cu" "*.Mask") (remove_unused_layers no))
  (pad "" thru_hole circle (at 158.42 143.18) (size 1.5 1.5) (drill 0.9) (layers "*.Cu" "*.Mask") (remove_unused_layers no))
  (pad "" thru_hole circle (at 158.42 145.72) (size 1.5 1.5) (drill 0.9) (layers "*.Cu" "*.Mask") (remove_unused_layers no))
  (pad "" thru_hole circle (at 158.42 148.26) (size 1.5 1.5) (drill 0.9) (layers "*.Cu" "*.Mask") (remove_unused_layers no))
  (pad "" thru_hole circle (at 160.96 120.32) (size 1.5 1.5) (drill 0.9) (layers "*.Cu" "*.Mask") (remove_unused_layers no))
  (pad "" thru_hole circle (at 160.96 122.86) (size 1.5 1.5) (drill 0.9) (layers "*.Cu" "*.Mask") (remove_unused_layers no))
  (pad "" thru_hole circle (at 160.96 125.4) (size 1.5 1.5) (drill 0.9) (layers "*.Cu" "*.Mask") (remove_unused_layers no))
  (pad "" thru_hole circle (at 160.96 127.94) (size 1.5 1.5) (drill 0.9) (layers "*.Cu" "*.Mask") (remove_unused_layers no))
  (pad "" thru_hole circle (at 160.96 130.48) (size 1.5 1.5) (drill 0.9) (layers "*.Cu" "*.Mask") (remove_unused_layers no))
  (pad "" thru_hole circle (at 160.96 135.56) (size 1.5 1.5) (drill 0.9) (layers "*.Cu" "*.Mask") (remove_unused_layers no))
  (pad "" thru_hole circle (at 160.96 138.1) (size 1.5 1.5) (drill 0.9) (layers "*.Cu" "*.Mask") (remove_unused_layers no))
  (pad "" thru_hole circle (at 160.96 140.64) (size 1.5 1.5) (drill 0.9) (layers "*.Cu" "*.Mask") (remove_unused_layers no))
  (pad "" thru_hole circle (at 160.96 143.18) (size 1.5 1.5) (drill 0.9) (layers "*.Cu" "*.Mask") (remove_unused_layers no))
  (pad "" thru_hole circle (at 160.96 145.72) (size 1.5 1.5) (drill 0.9) (layers "*.Cu" "*.Mask") (remove_unused_layers no))
  (pad "" thru_hole circle (at 160.96 148.26) (size 1.5 1.5) (drill 0.9) (layers "*.Cu" "*.Mask") (remove_unused_layers no))
  (pad "" thru_hole circle (at 163.5 120.32) (size 1.5 1.5) (drill 0.9) (layers "*.Cu" "*.Mask") (remove_unused_layers no))
  (pad "" thru_hole circle (at 163.5 122.86) (size 1.5 1.5) (drill 0.9) (layers "*.Cu" "*.Mask") (remove_unused_layers no))
  (pad "" thru_hole circle (at 163.5 125.4) (size 1.5 1.5) (drill 0.9) (layers "*.Cu" "*.Mask") (remove_unused_layers no))
  (pad "" thru_hole circle (at 163.5 127.94) (size 1.5 1.5) (drill 0.9) (layers "*.Cu" "*.Mask") (remove_unused_layers no))
  (pad "" thru_hole circle (at 163.5 130.48) (size 1.5 1.5) (drill 0.9) (layers "*.Cu" "*.Mask") (remove_unused_layers no))
  (pad "" thru_hole circle (at 163.5 135.56) (size 1.5 1.5) (drill 0.9) (layers "*.Cu" "*.Mask") (remove_unused_layers no))
  (pad "" thru_hole circle (at 163.5 138.1) (size 1.5 1.5) (drill 0.9) (layers "*.Cu" "*.Mask") (remove_unused_layers no))
  (pad "" thru_hole circle (at 163.5 140.64) (size 1.5 1.5) (drill 0.9) (layers "*.Cu" "*.Mask") (remove_unused_layers no))
  (pad "" thru_hole circle (at 163.5 143.18) (size 1.5 1.5) (drill 0.9) (layers "*.Cu" "*.Mask") (remove_unused_layers no))
  (pad "" thru_hole circle (at 163.5 145.72) (size 1.5 1.5) (drill 0.9) (layers "*.Cu" "*.Mask") (remove_unused_layers no))
  (pad "" thru_hole circle (at 163.5 148.26) (size 1.5 1.5) (drill 0.9) (layers "*.Cu" "*.Mask") (remove_unused_layers no))
  (pad "" thru_hole circle (at 166.04 120.32) (size 1.5 1.5) (drill 0.9) (layers "*.Cu" "*.Mask") (remove_unused_layers no))
  (pad "" thru_hole circle (at 166.04 122.86) (size 1.5 1.5) (drill 0.9) (layers "*.Cu" "*.Mask") (remove_unused_layers no))
  (pad "" thru_hole circle (at 166.04 125.4) (size 1.5 1.5) (drill 0.9) (layers "*.Cu" "*.Mask") (remove_unused_layers no))
  (pad "" thru_hole circle (at 166.04 127.94) (size 1.5 1.5) (drill 0.9) (layers "*.Cu" "*.Mask") (remove_unused_layers no))
  (pad "" thru_hole circle (at 166.04 130.48) (size 1.5 1.5) (drill 0.9) (layers "*.Cu" "*.Mask") (remove_unused_layers no))
  (pad "" thru_hole circle (at 166.04 133.02) (size 1.5 1.5) (drill 0.9) (layers "*.Cu" "*.Mask") (remove_unused_layers no))
  (pad "" thru_hole circle (at 166.04 135.56) (size 1.5 1.5) (drill 0.9) (layers "*.Cu" "*.Mask") (remove_unused_layers no))
  (pad "" thru_hole circle (at 166.04 138.1) (size 1.5 1.5) (drill 0.9) (layers "*.Cu" "*.Mask") (remove_unused_layers no))
  (pad "" thru_hole circle (at 166.04 140.64) (size 1.5 1.5) (drill 0.9) (layers "*.Cu" "*.Mask") (remove_unused_layers no))
  (pad "" thru_hole circle (at 166.04 143.18) (size 1.5 1.5) (drill 0.9) (layers "*.Cu" "*.Mask") (remove_unused_layers no))
  (pad "" thru_hole circle (at 166.04 145.72) (size 1.5 1.5) (drill 0.9) (layers "*.Cu" "*.Mask") (remove_unused_layers no))
  (pad "" thru_hole circle (at 166.04 148.26) (size 1.5 1.5) (drill 0.9) (layers "*.Cu" "*.Mask") (remove_unused_layers no)))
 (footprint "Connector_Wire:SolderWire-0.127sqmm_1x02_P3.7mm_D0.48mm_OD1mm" (layer "F.Cu") (at 153.34 140.64)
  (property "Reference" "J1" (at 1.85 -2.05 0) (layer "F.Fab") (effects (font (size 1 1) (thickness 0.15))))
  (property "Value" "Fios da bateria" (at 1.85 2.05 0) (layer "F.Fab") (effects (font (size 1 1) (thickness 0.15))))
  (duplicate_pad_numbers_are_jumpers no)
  (pad "1" thru_hole roundrect (at 0 0) (size 1.7 1.7) (drill 0.7) (layers "*.Cu" "*.Mask") (remove_unused_layers no)
   (roundrect_rratio 0.147059) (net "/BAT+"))
  (pad "2" thru_hole circle (at 3.7 0) (size 1.7 1.7) (drill 0.7) (layers "*.Cu" "*.Mask") (remove_unused_layers no) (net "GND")))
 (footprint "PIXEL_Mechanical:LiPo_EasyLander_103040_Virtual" (layer "B.Cu") (at 134 125)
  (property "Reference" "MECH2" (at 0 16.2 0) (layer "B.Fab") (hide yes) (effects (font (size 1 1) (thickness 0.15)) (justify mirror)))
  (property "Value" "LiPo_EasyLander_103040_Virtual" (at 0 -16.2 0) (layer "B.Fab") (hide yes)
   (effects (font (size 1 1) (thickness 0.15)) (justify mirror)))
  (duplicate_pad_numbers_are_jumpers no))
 (gr_arc (start 100 101) (mid 100.292893 100.292893) (end 101 100) (stroke (width 0.1) (type default)) (layer "Edge.Cuts"))
 (gr_line (start 100 149) (end 100 101) (stroke (width 0.1) (type default)) (layer "Edge.Cuts"))
 (gr_line (start 101 100) (end 169 100) (stroke (width 0.1) (type default)) (layer "Edge.Cuts"))
 (gr_arc (start 101 150) (mid 100.292893 149.707106) (end 100 149) (stroke (width 0.1) (type default)) (layer "Edge.Cuts"))
 (gr_arc (start 169 100) (mid 169.707106 100.292893) (end 170 101) (stroke (width 0.1) (type default)) (layer "Edge.Cuts"))
 (gr_line (start 169 150) (end 101 150) (stroke (width 0.1) (type default)) (layer "Edge.Cuts"))
 (gr_line (start 170 101) (end 170 149) (stroke (width 0.1) (type default)) (layer "Edge.Cuts"))
 (gr_arc (start 170 149) (mid 169.707106 149.707106) (end 169 150) (stroke (width 0.1) (type default)) (layer "Edge.Cuts"))
 (segment (start 110.16 123.4) (end 110.16 127.94) (width 0.4) (layer "F.Cu") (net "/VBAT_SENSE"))
 (segment (start 107.62 123.4) (end 110.16 123.4) (width 0.4) (layer "F.Cu") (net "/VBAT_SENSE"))
 (segment (start 105.08 127.94) (end 110.16 127.94) (width 0.4) (layer "F.Cu") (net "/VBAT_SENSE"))
 (segment (start 107.62 120.32) (end 107.62 123.4) (width 0.4) (layer "F.Cu") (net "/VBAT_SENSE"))
 (segment (start 110.16 135.56) (end 110.16 148.9) (width 0.6) (layer "B.Cu") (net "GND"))
 (segment (start 130.479998 115.24) (end 132.6 115.24) (width 0.6) (layer "B.Cu") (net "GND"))
 (segment (start 132.6 115.24) (end 132.6 148.9) (width 0.6) (layer "B.Cu") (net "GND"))
 (segment (start 100.9 148.9) (end 157.04 148.9) (width 0.6) (layer "B.Cu") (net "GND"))
 (segment (start 157.04 148.9) (end 157.04 140.64) (width 0.6) (layer "B.Cu") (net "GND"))
 (segment (start 100.9 107.62) (end 100.9 148.9) (width 0.6) (layer "B.Cu") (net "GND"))
 (segment (start 102.54 107.62) (end 100.9 107.62) (width 0.6) (layer "B.Cu") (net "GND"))
 (segment (start 102.54 112.7) (end 102.54 135.56) (width 0.5) (layer "F.Cu") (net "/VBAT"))
 (segment (start 105.08 145) (end 137.46 145) (width 0.5) (layer "F.Cu") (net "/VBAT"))
 (segment (start 137.46 145) (end 137.46 147.5) (width 0.5) (layer "F.Cu") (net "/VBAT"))
 (segment (start 105.08 135.56) (end 105.08 145) (width 0.5) (layer "F.Cu") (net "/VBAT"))
 (segment (start 102.54 135.56) (end 105.08 135.56) (width 0.5) (layer "F.Cu") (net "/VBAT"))
 (segment (start 130.479998 117.78) (end 130.479999 145) (width 0.5) (layer "F.Cu") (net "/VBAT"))
 (segment (start 112.7 120.32) (end 112.7 125.94) (width 0.4) (layer "F.Cu") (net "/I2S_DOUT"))
 (segment (start 128.4 125.94) (end 128.4 107.62) (width 0.4) (layer "F.Cu") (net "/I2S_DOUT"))
 (segment (start 128.4 107.62) (end 130.479998 107.62) (width 0.4) (layer "F.Cu") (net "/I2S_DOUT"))
 (segment (start 112.7 125.94) (end 128.4 125.94) (width 0.4) (layer "F.Cu") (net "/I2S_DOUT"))
 (segment (start 115.24 120.32) (end 115.24 124.4) (width 0.4) (layer "F.Cu") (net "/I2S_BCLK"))
 (segment (start 127.2 105.08) (end 130.479998 105.08) (width 0.4) (layer "F.Cu") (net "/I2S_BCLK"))
 (segment (start 115.24 124.4) (end 127.2 124.4) (width 0.4) (layer "F.Cu") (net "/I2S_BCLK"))
 (segment (start 127.2 124.4) (end 127.2 105.08) (width 0.4) (layer "F.Cu") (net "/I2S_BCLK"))
 (segment (start 126 102.54) (end 130.479998 102.54) (width 0.4) (layer "F.Cu") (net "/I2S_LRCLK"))
 (segment (start 117.78 120.32) (end 117.78 122.86) (width 0.4) (layer "F.Cu") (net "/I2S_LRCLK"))
 (segment (start 126 122.86) (end 126 102.54) (width 0.4) (layer "F.Cu") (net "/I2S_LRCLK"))
 (segment (start 117.78 122.86) (end 126 122.86) (width 0.4) (layer "F.Cu") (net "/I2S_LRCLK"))
 (segment (start 153.34 140.64) (end 153.34 143) (width 0.5) (layer "F.Cu") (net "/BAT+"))
 (segment (start 153.34 143) (end 140 143) (width 0.5) (layer "F.Cu") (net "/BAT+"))
 (segment (start 140 143) (end 140 147.5) (width 0.5) (layer "F.Cu") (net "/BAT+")))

